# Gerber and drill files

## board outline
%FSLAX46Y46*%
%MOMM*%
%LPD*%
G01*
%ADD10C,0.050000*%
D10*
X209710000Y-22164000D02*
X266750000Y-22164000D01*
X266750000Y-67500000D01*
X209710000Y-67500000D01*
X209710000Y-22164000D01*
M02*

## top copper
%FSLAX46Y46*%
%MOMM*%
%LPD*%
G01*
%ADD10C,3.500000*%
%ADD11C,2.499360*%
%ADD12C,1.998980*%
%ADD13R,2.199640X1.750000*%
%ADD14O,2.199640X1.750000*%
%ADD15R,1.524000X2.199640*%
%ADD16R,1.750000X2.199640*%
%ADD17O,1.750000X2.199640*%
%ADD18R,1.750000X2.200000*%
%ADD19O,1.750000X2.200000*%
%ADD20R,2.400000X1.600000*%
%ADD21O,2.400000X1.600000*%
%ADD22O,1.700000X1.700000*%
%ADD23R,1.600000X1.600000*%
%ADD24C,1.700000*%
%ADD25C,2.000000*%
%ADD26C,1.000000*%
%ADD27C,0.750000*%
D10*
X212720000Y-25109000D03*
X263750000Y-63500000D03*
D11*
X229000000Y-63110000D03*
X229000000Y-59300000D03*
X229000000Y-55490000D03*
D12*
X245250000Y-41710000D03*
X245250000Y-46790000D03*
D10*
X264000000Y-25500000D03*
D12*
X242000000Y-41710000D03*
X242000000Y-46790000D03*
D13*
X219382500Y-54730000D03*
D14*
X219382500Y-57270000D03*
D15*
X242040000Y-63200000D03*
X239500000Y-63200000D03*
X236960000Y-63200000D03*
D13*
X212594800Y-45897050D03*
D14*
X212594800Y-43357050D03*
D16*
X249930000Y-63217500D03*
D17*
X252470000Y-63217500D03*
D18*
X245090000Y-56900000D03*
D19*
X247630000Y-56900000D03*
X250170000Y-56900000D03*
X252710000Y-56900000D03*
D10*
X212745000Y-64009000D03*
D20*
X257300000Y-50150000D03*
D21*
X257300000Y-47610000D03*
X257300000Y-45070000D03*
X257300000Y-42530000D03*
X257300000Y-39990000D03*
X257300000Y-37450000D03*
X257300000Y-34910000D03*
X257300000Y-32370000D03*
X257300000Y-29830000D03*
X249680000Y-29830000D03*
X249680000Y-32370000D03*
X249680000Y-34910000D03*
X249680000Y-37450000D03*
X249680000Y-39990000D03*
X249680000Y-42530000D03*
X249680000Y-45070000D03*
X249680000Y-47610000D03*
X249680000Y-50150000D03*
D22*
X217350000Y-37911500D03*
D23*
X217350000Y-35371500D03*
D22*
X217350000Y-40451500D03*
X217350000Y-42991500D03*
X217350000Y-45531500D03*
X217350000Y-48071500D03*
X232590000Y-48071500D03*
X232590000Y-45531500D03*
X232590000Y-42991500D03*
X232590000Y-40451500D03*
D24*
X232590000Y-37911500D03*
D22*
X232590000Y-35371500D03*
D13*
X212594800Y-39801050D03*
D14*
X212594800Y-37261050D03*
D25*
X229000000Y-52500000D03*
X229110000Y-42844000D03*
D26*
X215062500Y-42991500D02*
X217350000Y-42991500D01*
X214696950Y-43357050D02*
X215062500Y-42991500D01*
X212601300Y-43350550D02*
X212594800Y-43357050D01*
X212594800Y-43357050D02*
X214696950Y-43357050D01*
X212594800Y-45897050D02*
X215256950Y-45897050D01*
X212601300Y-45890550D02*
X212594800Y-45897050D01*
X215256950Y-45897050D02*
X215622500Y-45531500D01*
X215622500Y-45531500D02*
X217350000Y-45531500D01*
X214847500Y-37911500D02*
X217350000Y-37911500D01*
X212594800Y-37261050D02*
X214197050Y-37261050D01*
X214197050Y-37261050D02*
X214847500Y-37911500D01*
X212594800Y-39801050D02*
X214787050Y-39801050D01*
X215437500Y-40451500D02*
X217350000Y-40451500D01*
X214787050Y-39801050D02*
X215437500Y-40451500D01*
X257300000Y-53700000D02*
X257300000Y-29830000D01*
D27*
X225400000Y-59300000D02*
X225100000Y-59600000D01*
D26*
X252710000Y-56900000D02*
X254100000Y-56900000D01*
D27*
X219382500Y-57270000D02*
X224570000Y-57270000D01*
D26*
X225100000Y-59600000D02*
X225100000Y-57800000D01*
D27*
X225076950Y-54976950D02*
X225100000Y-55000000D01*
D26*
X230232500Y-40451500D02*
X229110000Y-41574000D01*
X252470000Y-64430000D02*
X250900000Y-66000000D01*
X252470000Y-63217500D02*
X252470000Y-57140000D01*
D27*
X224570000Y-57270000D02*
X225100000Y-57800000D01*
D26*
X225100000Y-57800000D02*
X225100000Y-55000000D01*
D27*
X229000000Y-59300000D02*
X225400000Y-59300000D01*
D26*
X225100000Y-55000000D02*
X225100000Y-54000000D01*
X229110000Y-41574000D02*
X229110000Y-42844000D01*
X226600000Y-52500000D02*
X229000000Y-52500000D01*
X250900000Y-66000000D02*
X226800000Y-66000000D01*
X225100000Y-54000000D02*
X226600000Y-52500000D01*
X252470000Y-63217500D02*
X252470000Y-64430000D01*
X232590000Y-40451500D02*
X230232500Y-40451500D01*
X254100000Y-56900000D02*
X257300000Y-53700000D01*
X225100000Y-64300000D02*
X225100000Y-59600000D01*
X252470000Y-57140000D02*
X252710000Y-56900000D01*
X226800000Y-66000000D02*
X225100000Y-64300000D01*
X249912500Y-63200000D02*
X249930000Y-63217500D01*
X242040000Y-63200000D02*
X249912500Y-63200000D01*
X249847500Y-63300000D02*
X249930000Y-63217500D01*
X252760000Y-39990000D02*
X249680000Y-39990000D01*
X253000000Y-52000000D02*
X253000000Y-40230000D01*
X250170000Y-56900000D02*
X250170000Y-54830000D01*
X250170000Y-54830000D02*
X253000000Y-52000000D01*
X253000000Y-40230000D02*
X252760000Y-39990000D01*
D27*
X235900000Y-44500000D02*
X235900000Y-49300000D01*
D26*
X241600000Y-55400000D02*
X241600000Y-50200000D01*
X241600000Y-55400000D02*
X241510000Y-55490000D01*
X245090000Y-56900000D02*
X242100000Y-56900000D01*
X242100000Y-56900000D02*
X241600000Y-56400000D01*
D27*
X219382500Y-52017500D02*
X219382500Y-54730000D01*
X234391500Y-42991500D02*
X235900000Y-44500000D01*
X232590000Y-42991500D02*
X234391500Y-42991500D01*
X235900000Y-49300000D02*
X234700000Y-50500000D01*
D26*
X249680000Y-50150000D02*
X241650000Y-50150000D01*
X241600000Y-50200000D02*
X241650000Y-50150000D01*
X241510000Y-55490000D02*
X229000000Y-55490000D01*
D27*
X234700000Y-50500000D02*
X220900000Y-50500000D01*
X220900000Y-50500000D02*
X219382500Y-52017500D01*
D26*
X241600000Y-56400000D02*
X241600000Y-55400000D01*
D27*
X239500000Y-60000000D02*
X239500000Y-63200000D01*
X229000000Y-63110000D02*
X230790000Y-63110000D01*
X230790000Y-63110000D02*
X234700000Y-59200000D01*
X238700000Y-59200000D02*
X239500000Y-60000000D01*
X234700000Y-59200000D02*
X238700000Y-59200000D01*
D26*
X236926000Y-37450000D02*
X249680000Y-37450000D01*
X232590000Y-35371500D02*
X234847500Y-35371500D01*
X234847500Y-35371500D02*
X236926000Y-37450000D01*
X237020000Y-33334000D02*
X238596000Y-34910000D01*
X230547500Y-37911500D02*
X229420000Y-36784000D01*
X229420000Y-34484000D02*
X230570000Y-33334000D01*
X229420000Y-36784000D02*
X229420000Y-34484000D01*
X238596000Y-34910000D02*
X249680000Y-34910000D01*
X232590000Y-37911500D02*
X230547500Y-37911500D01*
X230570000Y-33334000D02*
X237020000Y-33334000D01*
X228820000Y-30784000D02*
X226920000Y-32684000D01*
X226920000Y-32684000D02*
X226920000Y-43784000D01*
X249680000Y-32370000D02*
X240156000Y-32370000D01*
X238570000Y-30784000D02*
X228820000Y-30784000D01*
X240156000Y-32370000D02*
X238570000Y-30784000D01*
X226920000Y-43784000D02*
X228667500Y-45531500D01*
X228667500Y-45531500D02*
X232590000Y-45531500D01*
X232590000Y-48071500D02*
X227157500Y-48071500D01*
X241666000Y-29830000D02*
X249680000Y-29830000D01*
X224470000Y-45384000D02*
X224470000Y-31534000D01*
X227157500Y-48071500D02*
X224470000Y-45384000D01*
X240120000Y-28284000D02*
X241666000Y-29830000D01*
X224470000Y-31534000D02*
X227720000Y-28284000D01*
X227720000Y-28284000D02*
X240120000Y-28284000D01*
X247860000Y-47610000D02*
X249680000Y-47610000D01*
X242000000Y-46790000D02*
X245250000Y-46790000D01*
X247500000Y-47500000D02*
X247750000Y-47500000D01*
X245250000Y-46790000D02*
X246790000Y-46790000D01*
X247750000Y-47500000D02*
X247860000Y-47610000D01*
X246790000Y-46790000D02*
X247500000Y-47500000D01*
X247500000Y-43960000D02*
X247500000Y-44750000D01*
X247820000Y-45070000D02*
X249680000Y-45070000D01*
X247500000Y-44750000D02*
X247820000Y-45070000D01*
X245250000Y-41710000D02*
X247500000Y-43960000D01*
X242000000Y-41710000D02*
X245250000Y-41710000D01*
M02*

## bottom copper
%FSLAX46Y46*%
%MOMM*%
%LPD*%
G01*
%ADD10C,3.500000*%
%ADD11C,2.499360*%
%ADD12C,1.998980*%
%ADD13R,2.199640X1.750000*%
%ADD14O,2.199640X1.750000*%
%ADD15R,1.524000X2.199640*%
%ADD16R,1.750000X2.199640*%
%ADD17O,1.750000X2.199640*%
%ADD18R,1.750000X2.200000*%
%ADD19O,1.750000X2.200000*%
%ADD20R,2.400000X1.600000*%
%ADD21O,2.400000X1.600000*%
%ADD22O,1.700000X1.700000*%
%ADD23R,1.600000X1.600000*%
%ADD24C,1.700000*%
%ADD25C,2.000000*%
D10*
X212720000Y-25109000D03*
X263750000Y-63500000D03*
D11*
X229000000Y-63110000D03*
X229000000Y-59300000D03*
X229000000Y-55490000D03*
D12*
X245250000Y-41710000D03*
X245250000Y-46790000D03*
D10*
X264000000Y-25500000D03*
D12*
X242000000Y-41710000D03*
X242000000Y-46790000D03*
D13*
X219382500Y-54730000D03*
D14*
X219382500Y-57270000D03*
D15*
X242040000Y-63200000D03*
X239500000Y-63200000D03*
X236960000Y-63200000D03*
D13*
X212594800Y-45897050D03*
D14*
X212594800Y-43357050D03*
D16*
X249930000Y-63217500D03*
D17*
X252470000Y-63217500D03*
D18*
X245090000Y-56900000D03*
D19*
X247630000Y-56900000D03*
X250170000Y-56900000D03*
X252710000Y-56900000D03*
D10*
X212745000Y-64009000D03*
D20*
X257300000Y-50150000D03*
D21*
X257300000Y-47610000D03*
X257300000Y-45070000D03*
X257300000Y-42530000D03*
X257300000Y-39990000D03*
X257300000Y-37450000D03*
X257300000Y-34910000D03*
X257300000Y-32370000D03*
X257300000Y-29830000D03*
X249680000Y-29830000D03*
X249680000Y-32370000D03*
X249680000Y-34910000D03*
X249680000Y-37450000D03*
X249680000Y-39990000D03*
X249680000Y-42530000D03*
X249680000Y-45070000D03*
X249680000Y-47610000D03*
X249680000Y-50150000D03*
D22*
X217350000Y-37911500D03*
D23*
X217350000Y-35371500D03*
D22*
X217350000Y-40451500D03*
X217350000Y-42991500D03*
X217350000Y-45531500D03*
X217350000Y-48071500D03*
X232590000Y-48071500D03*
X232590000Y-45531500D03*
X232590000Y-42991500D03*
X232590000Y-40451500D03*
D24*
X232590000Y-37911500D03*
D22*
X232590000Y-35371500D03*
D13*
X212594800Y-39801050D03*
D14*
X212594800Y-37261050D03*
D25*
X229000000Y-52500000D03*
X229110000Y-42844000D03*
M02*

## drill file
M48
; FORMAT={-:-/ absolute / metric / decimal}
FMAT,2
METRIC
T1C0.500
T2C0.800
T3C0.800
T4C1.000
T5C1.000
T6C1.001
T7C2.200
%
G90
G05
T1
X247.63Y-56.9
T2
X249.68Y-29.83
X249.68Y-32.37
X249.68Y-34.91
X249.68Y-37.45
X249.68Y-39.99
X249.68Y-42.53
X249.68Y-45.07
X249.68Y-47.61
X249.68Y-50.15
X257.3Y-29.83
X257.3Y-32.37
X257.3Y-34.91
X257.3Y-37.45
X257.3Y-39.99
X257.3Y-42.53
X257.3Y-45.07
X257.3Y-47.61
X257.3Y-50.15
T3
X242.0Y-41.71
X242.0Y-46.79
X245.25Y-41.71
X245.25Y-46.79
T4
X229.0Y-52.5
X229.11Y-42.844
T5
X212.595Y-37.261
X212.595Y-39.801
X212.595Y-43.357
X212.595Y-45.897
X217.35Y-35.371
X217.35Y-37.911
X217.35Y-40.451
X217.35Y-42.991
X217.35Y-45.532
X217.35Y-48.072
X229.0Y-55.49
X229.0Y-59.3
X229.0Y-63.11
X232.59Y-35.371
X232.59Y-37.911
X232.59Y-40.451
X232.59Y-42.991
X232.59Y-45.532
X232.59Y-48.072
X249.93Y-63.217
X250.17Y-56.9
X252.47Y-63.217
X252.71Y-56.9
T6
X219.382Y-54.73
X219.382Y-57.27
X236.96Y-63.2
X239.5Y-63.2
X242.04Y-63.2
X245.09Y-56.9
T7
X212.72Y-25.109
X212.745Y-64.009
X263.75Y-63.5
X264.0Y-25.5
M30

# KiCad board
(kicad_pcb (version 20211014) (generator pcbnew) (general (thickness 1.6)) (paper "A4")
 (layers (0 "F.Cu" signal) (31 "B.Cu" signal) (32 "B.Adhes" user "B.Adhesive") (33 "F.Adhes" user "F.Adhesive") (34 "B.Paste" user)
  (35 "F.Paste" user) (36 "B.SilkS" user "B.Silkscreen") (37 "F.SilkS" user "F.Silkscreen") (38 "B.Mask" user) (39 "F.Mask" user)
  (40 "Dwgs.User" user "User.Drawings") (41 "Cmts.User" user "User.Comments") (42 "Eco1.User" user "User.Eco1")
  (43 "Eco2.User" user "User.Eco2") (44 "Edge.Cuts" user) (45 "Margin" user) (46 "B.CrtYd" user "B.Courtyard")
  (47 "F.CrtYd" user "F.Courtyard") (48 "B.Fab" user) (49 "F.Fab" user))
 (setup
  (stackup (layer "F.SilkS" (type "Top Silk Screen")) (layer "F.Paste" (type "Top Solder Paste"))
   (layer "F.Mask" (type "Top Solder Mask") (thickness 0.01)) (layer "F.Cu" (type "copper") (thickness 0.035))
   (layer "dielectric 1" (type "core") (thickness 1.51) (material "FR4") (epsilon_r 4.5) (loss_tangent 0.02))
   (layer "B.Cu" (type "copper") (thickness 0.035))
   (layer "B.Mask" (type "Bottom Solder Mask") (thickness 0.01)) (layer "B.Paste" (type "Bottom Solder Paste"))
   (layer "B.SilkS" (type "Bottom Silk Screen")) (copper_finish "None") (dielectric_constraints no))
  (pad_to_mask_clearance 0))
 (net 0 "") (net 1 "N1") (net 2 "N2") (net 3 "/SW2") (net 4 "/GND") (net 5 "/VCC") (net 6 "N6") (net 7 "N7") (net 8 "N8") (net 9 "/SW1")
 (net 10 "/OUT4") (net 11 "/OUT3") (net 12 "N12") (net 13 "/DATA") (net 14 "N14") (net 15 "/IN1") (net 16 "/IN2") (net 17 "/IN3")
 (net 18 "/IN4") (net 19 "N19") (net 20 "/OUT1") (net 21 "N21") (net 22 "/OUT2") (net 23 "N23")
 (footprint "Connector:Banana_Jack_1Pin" (layer "F.Cu") (at 212.72 25.109)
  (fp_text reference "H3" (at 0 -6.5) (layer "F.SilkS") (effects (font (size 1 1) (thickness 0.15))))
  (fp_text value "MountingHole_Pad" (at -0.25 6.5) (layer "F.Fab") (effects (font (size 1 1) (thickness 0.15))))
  (pad "1" thru_hole circle (at 0 0) (size 3.5 3.5) (drill 2.2) (layers *.Cu *.Mask) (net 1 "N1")))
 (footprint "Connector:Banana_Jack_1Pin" (layer "F.Cu") (at 263.75 63.5)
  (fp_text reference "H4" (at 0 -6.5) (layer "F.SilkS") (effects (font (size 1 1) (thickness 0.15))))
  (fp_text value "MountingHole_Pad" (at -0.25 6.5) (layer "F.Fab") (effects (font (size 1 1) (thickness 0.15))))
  (pad "1" thru_hole circle (at 0 0) (size 3.5 3.5) (drill 2.2) (layers *.Cu *.Mask) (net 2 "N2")))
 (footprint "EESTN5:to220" (layer "F.Cu") (at 229 59.3 90)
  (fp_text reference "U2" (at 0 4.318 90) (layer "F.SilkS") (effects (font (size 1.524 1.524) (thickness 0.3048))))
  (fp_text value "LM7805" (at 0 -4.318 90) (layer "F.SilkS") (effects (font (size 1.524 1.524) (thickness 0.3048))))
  (pad "1" thru_hole circle locked (at -3.81 0 90) (size 2.49936 2.49936) (drill 1) (layers *.Cu *.Mask "F.SilkS") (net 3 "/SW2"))
  (pad "2" thru_hole circle locked (at 0 0 90) (size 2.49936 2.49936) (drill 1) (layers *.Cu *.Mask "F.SilkS") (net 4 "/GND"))
  (pad "3" thru_hole circle locked (at 3.81 0 90) (size 2.49936 2.49936) (drill 1) (layers *.Cu *.Mask "F.SilkS") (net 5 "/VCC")))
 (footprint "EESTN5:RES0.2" (layer "F.Cu") (at 245.25 44.25 -90)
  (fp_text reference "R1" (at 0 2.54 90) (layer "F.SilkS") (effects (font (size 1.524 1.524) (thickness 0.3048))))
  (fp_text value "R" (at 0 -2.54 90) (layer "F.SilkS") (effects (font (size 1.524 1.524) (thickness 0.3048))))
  (pad "1" thru_hole circle locked (at -2.54 0 270) (size 1.99898 1.99898) (drill 0.8001) (layers *.Cu *.Mask "F.SilkS") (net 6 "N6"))
  (pad "2" thru_hole circle locked (at 2.54 0 270) (size 1.99898 1.99898) (drill 0.8001) (layers *.Cu *.Mask "F.SilkS") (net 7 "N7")))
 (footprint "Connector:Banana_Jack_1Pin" (layer "F.Cu") (at 264 25.5)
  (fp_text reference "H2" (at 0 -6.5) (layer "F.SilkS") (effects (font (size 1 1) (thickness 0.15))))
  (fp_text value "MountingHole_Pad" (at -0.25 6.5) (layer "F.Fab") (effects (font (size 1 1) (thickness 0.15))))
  (pad "1" thru_hole circle (at 0 0) (size 3.5 3.5) (drill 2.2) (layers *.Cu *.Mask) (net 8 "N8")))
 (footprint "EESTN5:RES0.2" (layer "F.Cu") (at 242 44.25 -90)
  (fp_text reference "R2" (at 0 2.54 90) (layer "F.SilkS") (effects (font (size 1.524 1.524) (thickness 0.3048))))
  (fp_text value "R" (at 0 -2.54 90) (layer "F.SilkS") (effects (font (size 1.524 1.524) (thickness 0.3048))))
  (pad "1" thru_hole circle locked (at -2.54 0 270) (size 1.99898 1.99898) (drill 0.8001) (layers *.Cu *.Mask "F.SilkS") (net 6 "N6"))
  (pad "2" thru_hole circle locked (at 2.54 0 270) (size 1.99898 1.99898) (drill 0.8001) (layers *.Cu *.Mask "F.SilkS") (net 7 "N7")))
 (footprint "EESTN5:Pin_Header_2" (layer "F.Cu") (at 219.7 56 -90)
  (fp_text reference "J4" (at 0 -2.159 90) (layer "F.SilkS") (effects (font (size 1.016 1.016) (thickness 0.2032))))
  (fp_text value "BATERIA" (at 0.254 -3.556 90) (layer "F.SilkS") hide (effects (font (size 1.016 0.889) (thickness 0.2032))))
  (pad "1" thru_hole rect locked (at -1.27 0.3175 270) (size 1.75 2.19964) (drill 1.00076) (layers *.Cu *.Mask "F.SilkS") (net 5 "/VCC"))
  (pad "2" thru_hole oval locked (at 1.27 0.3175 270) (size 1.75 2.19964) (drill 1.00076) (layers *.Cu *.Mask "F.SilkS") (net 4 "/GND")))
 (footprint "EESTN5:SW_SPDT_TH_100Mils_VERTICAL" (layer "F.Cu") (at 239.5 63.2 180)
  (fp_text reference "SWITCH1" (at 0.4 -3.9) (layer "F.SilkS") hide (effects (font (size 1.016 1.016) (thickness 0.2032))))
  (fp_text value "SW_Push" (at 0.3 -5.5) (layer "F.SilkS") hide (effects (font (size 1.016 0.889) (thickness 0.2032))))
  (pad "1" thru_hole rect locked (at -2.54 0 180) (size 1.524 2.19964) (drill 1.00076) (layers *.Cu *.Mask "F.SilkS") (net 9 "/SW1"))
  (pad "2" thru_hole rect locked (at 0 0 180) (size 1.524 2.19964) (drill 1.00076) (layers *.Cu *.Mask "F.SilkS") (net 3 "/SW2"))
  (pad "3" thru_hole rect locked (at 2.54 0 180) (size 1.524 2.19964) (drill 1.00076) (layers *.Cu *.Mask "F.SilkS")))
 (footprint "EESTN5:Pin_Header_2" (layer "F.Cu") (at 212.2773 44.62705 90)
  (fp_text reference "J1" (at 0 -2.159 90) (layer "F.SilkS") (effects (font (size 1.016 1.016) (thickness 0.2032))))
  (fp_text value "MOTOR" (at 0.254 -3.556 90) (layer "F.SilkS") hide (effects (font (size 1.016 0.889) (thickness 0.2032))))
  (pad "1" thru_hole rect locked (at -1.27 0.3175 90) (size 1.75 2.19964) (drill 1) (layers *.Cu *.Mask "F.SilkS") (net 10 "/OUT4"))
  (pad "2" thru_hole oval locked (at 1.27 0.3175 90) (size 1.75 2.19964) (drill 1) (layers *.Cu *.Mask "F.SilkS") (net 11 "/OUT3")))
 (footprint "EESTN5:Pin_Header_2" (layer "F.Cu") (at 251.2 62.9)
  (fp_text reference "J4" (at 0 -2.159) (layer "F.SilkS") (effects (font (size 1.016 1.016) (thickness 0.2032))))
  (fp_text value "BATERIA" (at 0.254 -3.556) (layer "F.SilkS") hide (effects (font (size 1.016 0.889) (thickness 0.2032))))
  (pad "1" thru_hole rect locked (at -1.27 0.3175) (size 1.75 2.19964) (drill 1) (layers *.Cu *.Mask "F.SilkS") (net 9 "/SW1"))
  (pad "2" thru_hole oval locked (at 1.27 0.3175) (size 1.75 2.19964) (drill 1) (layers *.Cu *.Mask "F.SilkS") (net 4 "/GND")))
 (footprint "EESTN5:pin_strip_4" (layer "F.Cu") (at 248.9 56.9)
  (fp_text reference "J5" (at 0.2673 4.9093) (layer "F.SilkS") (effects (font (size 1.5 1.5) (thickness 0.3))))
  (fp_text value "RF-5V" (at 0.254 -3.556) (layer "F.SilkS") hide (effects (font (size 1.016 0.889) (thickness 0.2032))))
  (pad "1" thru_hole rect locked (at -3.81 0) (size 1.75 2.2) (drill 1.00076) (layers *.Cu *.Mask "F.SilkS") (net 5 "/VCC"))
  (pad "2" thru_hole oval locked (at -1.27 0) (size 1.75 2.2) (drill 0.5) (layers *.Cu *.Mask "F.SilkS") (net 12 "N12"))
  (pad "3" thru_hole oval locked (at 1.27 0) (size 1.75 2.2) (drill 1) (layers *.Cu *.Mask "F.SilkS") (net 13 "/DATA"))
  (pad "4" thru_hole oval locked (at 3.81 0) (size 1.75 2.2) (drill 1) (layers *.Cu *.Mask "F.SilkS") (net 4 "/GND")))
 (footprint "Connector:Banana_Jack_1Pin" (layer "F.Cu") (at 212.745 64.009)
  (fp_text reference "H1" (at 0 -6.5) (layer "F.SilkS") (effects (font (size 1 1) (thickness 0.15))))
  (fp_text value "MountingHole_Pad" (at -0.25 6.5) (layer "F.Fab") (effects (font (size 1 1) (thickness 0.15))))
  (pad "1" thru_hole circle (at 0 0) (size 3.5 3.5) (drill 2.2) (layers *.Cu *.Mask) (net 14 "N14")))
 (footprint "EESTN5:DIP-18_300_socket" (layer "F.Cu") (at 257.3 50.15 180)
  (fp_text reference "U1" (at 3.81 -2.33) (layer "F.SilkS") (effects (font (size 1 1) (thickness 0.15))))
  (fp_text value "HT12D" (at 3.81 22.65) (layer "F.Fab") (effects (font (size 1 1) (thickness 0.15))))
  (pad "1" thru_hole rect locked (at 0 0 180) (size 2.4 1.6) (drill 0.8) (layers *.Cu *.Mask) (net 4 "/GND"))
  (pad "2" thru_hole oval locked (at 0 2.54 180) (size 2.4 1.6) (drill 0.8) (layers *.Cu *.Mask) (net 4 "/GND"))
  (pad "3" thru_hole oval locked (at 0 5.08 180) (size 2.4 1.6) (drill 0.8) (layers *.Cu *.Mask) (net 4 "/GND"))
  (pad "4" thru_hole oval locked (at 0 7.62 180) (size 2.4 1.6) (drill 0.8) (layers *.Cu *.Mask) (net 4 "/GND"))
  (pad "5" thru_hole oval locked (at 0 10.16 180) (size 2.4 1.6) (drill 0.8) (layers *.Cu *.Mask) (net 4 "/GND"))
  (pad "6" thru_hole oval locked (at 0 12.7 180) (size 2.4 1.6) (drill 0.8) (layers *.Cu *.Mask) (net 4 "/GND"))
  (pad "7" thru_hole oval locked (at 0 15.24 180) (size 2.4 1.6) (drill 0.8) (layers *.Cu *.Mask) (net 4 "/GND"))
  (pad "8" thru_hole oval locked (at 0 17.78 180) (size 2.4 1.6) (drill 0.8) (layers *.Cu *.Mask) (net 4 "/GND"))
  (pad "9" thru_hole oval locked (at 0 20.32 180) (size 2.4 1.6) (drill 0.8) (layers *.Cu *.Mask) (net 4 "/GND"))
  (pad "10" thru_hole oval locked (at 7.62 20.32 180) (size 2.4 1.6) (drill 0.8) (layers *.Cu *.Mask) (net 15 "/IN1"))
  (pad "11" thru_hole oval locked (at 7.62 17.78 180) (size 2.4 1.6) (drill 0.8) (layers *.Cu *.Mask) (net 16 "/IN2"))
  (pad "12" thru_hole oval locked (at 7.62 15.24 180) (size 2.4 1.6) (drill 0.8) (layers *.Cu *.Mask) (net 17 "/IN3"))
  (pad "13" thru_hole oval locked (at 7.62 12.7 180) (size 2.4 1.6) (drill 0.8) (layers *.Cu *.Mask) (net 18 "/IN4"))
  (pad "14" thru_hole oval locked (at 7.62 10.16 180) (size 2.4 1.6) (drill 0.8) (layers *.Cu *.Mask) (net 13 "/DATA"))
  (pad "15" thru_hole oval locked (at 7.62 7.62 180) (size 2.4 1.6) (drill 0.8) (layers *.Cu *.Mask) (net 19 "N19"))
  (pad "16" thru_hole oval locked (at 7.62 5.08 180) (size 2.4 1.6) (drill 0.8) (layers *.Cu *.Mask) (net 6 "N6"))
  (pad "17" thru_hole oval locked (at 7.62 2.54 180) (size 2.4 1.6) (drill 0.8) (layers *.Cu *.Mask) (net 7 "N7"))
  (pad "18" thru_hole oval locked (at 7.62 0 180) (size 2.4 1.6) (drill 0.8) (layers *.Cu *.Mask) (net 5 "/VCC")))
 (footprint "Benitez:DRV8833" (layer "F.Cu") (at 217.35 35.3715)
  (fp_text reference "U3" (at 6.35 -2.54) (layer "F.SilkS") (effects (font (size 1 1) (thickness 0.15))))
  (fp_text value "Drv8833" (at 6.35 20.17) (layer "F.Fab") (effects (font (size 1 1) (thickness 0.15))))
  (pad "1" thru_hole oval (at 0 2.54) (size 1.7 1.7) (drill 1) (layers *.Cu *.Mask) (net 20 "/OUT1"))
  (pad "1" thru_hole rect (at 0 0) (size 1.6 1.6) (drill 1) (layers *.Cu *.Mask) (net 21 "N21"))
  (pad "3" thru_hole oval (at 0 5.08) (size 1.7 1.7) (drill 1) (layers *.Cu *.Mask "B.SilkS") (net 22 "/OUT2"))
  (pad "4" thru_hole oval (at 0 7.62) (size 1.7 1.7) (drill 1) (layers *.Cu *.Mask) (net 11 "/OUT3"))
  (pad "5" thru_hole oval (at 0 10.16) (size 1.7 1.7) (drill 1) (layers *.Cu *.Mask) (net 10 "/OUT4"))
  (pad "6" thru_hole oval (at 0 12.7) (size 1.7 1.7) (drill 1) (layers *.Cu *.Mask) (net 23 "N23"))
  (pad "7" thru_hole oval (at 15.24 12.7) (size 1.7 1.7) (drill 1) (layers *.Cu *.Mask) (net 15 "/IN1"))
  (pad "8" thru_hole oval (at 15.24 10.16) (size 1.7 1.7) (drill 1) (layers *.Cu *.Mask) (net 16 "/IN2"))
  (pad "9" thru_hole oval (at 15.24 7.62) (size 1.7 1.7) (drill 1) (layers *.Cu *.Mask) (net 5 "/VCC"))
  (pad "10" thru_hole oval (at 15.24 5.08) (size 1.7 1.7) (drill 1) (layers *.Cu *.Mask) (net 4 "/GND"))
  (pad "11" thru_hole circle (at 15.24 2.54) (size 1.7 1.7) (drill 1) (layers *.Cu *.Mask) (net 17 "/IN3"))
  (pad "12" thru_hole oval (at 15.24 0) (size 1.7 1.7) (drill 1) (layers *.Cu *.Mask) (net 18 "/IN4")))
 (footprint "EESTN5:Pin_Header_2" (layer "F.Cu") (at 212.2773 38.53105 90)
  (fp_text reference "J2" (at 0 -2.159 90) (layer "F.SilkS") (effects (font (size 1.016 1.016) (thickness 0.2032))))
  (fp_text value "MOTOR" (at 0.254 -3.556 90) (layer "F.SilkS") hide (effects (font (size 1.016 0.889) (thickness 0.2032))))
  (pad "1" thru_hole rect locked (at -1.27 0.3175 90) (size 1.75 2.19964) (drill 1) (layers *.Cu *.Mask "F.SilkS") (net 22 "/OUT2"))
  (pad "2" thru_hole oval locked (at 1.27 0.3175 90) (size 1.75 2.19964) (drill 1) (layers *.Cu *.Mask "F.SilkS") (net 20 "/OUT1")))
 (gr_rect (start 266.75 67.5) (end 209.71 22.164) (layer "Edge.Cuts") (width 0.05) (fill none))
 (segment (start 215.0625 42.9915) (end 217.35 42.9915) (width 1) (layer "F.Cu") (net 11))
 (segment (start 214.69695 43.35705) (end 215.0625 42.9915) (width 1) (layer "F.Cu") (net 11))
 (segment (start 212.6013 43.35055) (end 212.5948 43.35705) (width 1) (layer "F.Cu") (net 11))
 (segment (start 212.5948 43.35705) (end 214.69695 43.35705) (width 1) (layer "F.Cu") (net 11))
 (segment (start 212.5948 45.89705) (end 215.25695 45.89705) (width 1) (layer "F.Cu") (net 10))
 (segment (start 212.6013 45.89055) (end 212.5948 45.89705) (width 1) (layer "F.Cu") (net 10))
 (segment (start 215.25695 45.89705) (end 215.6225 45.5315) (width 1) (layer "F.Cu") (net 10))
 (segment (start 215.6225 45.5315) (end 217.35 45.5315) (width 1) (layer "F.Cu") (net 10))
 (segment (start 214.8475 37.9115) (end 217.35 37.9115) (width 1) (layer "F.Cu") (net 20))
 (segment (start 212.5948 37.26105) (end 214.19705 37.26105) (width 1) (layer "F.Cu") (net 20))
 (segment (start 214.19705 37.26105) (end 214.8475 37.9115) (width 1) (layer "F.Cu") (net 20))
 (segment (start 212.5948 39.80105) (end 214.78705 39.80105) (width 1) (layer "F.Cu") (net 22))
 (segment (start 215.4375 40.4515) (end 217.35 40.4515) (width 1) (layer "F.Cu") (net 22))
 (segment (start 214.78705 39.80105) (end 215.4375 40.4515) (width 1) (layer "F.Cu") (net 22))
 (segment (start 257.3 53.7) (end 257.3 29.83) (width 1) (layer "F.Cu") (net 4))
 (segment (start 225.4 59.3) (end 225.1 59.6) (width 0.75) (layer "F.Cu") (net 4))
 (segment (start 252.71 56.9) (end 254.1 56.9) (width 1) (layer "F.Cu") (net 4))
 (segment (start 219.3825 57.27) (end 224.57 57.27) (width 0.75) (layer "F.Cu") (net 4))
 (segment (start 225.1 59.6) (end 225.1 57.8) (width 1) (layer "F.Cu") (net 4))
 (segment (start 225.07695 54.97695) (end 225.1 55) (width 0.75) (layer "F.Cu") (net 4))
 (segment (start 230.2325 40.4515) (end 229.11 41.574) (width 1) (layer "F.Cu") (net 4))
 (segment (start 252.47 64.43) (end 250.9 66) (width 1) (layer "F.Cu") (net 4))
 (segment (start 252.47 63.2175) (end 252.47 57.14) (width 1) (layer "F.Cu") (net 4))
 (segment (start 224.57 57.27) (end 225.1 57.8) (width 0.75) (layer "F.Cu") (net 4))
 (segment (start 225.1 57.8) (end 225.1 55) (width 1) (layer "F.Cu") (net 4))
 (segment (start 229 59.3) (end 225.4 59.3) (width 0.75) (layer "F.Cu") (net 4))
 (segment (start 225.1 55) (end 225.1 54) (width 1) (layer "F.Cu") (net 4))
 (segment (start 229.11 41.574) (end 229.11 42.844) (width 1) (layer "F.Cu") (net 4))
 (segment (start 226.6 52.5) (end 229 52.5) (width 1) (layer "F.Cu") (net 4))
 (segment (start 250.9 66) (end 226.8 66) (width 1) (layer "F.Cu") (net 4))
 (segment (start 225.1 54) (end 226.6 52.5) (width 1) (layer "F.Cu") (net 4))
 (segment (start 252.47 63.2175) (end 252.47 64.43) (width 1) (layer "F.Cu") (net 4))
 (segment (start 232.59 40.4515) (end 230.2325 40.4515) (width 1) (layer "F.Cu") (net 4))
 (segment (start 254.1 56.9) (end 257.3 53.7) (width 1) (layer "F.Cu") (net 4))
 (segment (start 225.1 64.3) (end 225.1 59.6) (width 1) (layer "F.Cu") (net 4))
 (segment (start 252.47 57.14) (end 252.71 56.9) (width 1) (layer "F.Cu") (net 4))
 (segment (start 226.8 66) (end 225.1 64.3) (width 1) (layer "F.Cu") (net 4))
 (via (at 229 52.5) (size 2) (drill 1) (layers "F.Cu" "B.Cu") (free) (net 4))
 (via (at 229.11 42.844) (size 2) (drill 1) (layers "F.Cu" "B.Cu") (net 4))
 (segment (start 249.9125 63.2) (end 249.93 63.2175) (width 1) (layer "F.Cu") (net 9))
 (segment (start 242.04 63.2) (end 249.9125 63.2) (width 1) (layer "F.Cu") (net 9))
 (segment (start 249.8475 63.3) (end 249.93 63.2175) (width 1) (layer "F.Cu") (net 9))
 (segment (start 252.76 39.99) (end 249.68 39.99) (width 1) (layer "F.Cu") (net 13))
 (segment (start 253 52) (end 253 40.23) (width 1) (layer "F.Cu") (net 13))
 (segment (start 250.17 56.9) (end 250.17 54.83) (width 1) (layer "F.Cu") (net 13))
 (segment (start 250.17 54.83) (end 253 52) (width 1) (layer "F.Cu") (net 13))
 (segment (start 253 40.23) (end 252.76 39.99) (width 1) (layer "F.Cu") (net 13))
 (segment (start 235.9 44.5) (end 235.9 49.3) (width 0.75) (layer "F.Cu") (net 5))
 (segment (start 241.6 55.4) (end 241.6 50.2) (width 1) (layer "F.Cu") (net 5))
 (segment (start 241.6 55.4) (end 241.51 55.49) (width 1) (layer "F.Cu") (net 5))
 (segment (start 245.09 56.9) (end 242.1 56.9) (width 1) (layer "F.Cu") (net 5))
 (segment (start 242.1 56.9) (end 241.6 56.4) (width 1) (layer "F.Cu") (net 5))
 (segment (start 219.3825 52.0175) (end 219.3825 54.73) (width 0.75) (layer "F.Cu") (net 5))
 (segment (start 234.3915 42.9915) (end 235.9 44.5) (width 0.75) (layer "F.Cu") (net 5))
 (segment (start 232.59 42.9915) (end 234.3915 42.9915) (width 0.75) (layer "F.Cu") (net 5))
 (segment (start 235.9 49.3) (end 234.7 50.5) (width 0.75) (layer "F.Cu") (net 5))
 (segment (start 249.68 50.15) (end 241.65 50.15) (width 1) (layer "F.Cu") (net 5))
 (segment (start 241.6 50.2) (end 241.65 50.15) (width 1) (layer "F.Cu") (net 5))
 (segment (start 241.51 55.49) (end 229 55.49) (width 1) (layer "F.Cu") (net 5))
 (segment (start 234.7 50.5) (end 220.9 50.5) (width 0.75) (layer "F.Cu") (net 5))
 (segment (start 220.9 50.5) (end 219.3825 52.0175) (width 0.75) (layer "F.Cu") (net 5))
 (segment (start 241.6 56.4) (end 241.6 55.4) (width 1) (layer "F.Cu") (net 5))
 (segment (start 239.5 60) (end 239.5 63.2) (width 0.75) (layer "F.Cu") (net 3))
 (segment (start 229 63.11) (end 230.79 63.11) (width 0.75) (layer "F.Cu") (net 3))
 (segment (start 230.79 63.11) (end 234.7 59.2) (width 0.75) (layer "F.Cu") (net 3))
 (segment (start 238.7 59.2) (end 239.5 60) (width 0.75) (layer "F.Cu") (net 3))
 (segment (start 234.7 59.2) (end 238.7 59.2) (width 0.75) (layer "F.Cu") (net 3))
 (segment (start 236.926 37.45) (end 249.68 37.45) (width 1) (layer "F.Cu") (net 18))
 (segment (start 232.59 35.3715) (end 234.8475 35.3715) (width 1) (layer "F.Cu") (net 18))
 (segment (start 234.8475 35.3715) (end 236.926 37.45) (width 1) (layer "F.Cu") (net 18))
 (segment (start 237.02 33.334) (end 238.596 34.91) (width 1) (layer "F.Cu") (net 17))
 (segment (start 230.5475 37.9115) (end 229.42 36.784) (width 1) (layer "F.Cu") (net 17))
 (segment (start 229.42 34.484) (end 230.57 33.334) (width 1) (layer "F.Cu") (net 17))
 (segment (start 229.42 36.784) (end 229.42 34.484) (width 1) (layer "F.Cu") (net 17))
 (segment (start 238.596 34.91) (end 249.68 34.91) (width 1) (layer "F.Cu") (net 17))
 (segment (start 232.59 37.9115) (end 230.5475 37.9115) (width 1) (layer "F.Cu") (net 17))
 (segment (start 230.57 33.334) (end 237.02 33.334) (width 1) (layer "F.Cu") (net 17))
 (segment (start 228.82 30.784) (end 226.92 32.684) (width 1) (layer "F.Cu") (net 16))
 (segment (start 226.92 32.684) (end 226.92 43.784) (width 1) (layer "F.Cu") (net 16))
 (segment (start 249.68 32.37) (end 240.156 32.37) (width 1) (layer "F.Cu") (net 16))
 (segment (start 238.57 30.784) (end 228.82 30.784) (width 1) (layer "F.Cu") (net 16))
 (segment (start 240.156 32.37) (end 238.57 30.784) (width 1) (layer "F.Cu") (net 16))
 (segment (start 226.92 43.784) (end 228.6675 45.5315) (width 1) (layer "F.Cu") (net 16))
 (segment (start 228.6675 45.5315) (end 232.59 45.5315) (width 1) (layer "F.Cu") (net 16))
 (segment (start 232.59 48.0715) (end 227.1575 48.0715) (width 1) (layer "F.Cu") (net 15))
 (segment (start 241.666 29.83) (end 249.68 29.83) (width 1) (layer "F.Cu") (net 15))
 (segment (start 224.47 45.384) (end 224.47 31.534) (width 1) (layer "F.Cu") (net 15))
 (segment (start 227.1575 48.0715) (end 224.47 45.384) (width 1) (layer "F.Cu") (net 15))
 (segment (start 240.12 28.284) (end 241.666 29.83) (width 1) (layer "F.Cu") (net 15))
 (segment (start 224.47 31.534) (end 227.72 28.284) (width 1) (layer "F.Cu") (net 15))
 (segment (start 227.72 28.284) (end 240.12 28.284) (width 1) (layer "F.Cu") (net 15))
 (segment (start 247.86 47.61) (end 249.68 47.61) (width 1) (layer "F.Cu") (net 7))
 (segment (start 242 46.79) (end 245.25 46.79) (width 1) (layer "F.Cu") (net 7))
 (segment (start 247.5 47.5) (end 247.75 47.5) (width 1) (layer "F.Cu") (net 7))
 (segment (start 245.25 46.79) (end 246.79 46.79) (width 1) (layer "F.Cu") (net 7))
 (segment (start 247.75 47.5) (end 247.86 47.61) (width 1) (layer "F.Cu") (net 7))
 (segment (start 246.79 46.79) (end 247.5 47.5) (width 1) (layer "F.Cu") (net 7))
 (segment (start 247.5 43.96) (end 247.5 44.75) (width 1) (layer "F.Cu") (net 6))
 (segment (start 247.82 45.07) (end 249.68 45.07) (width 1) (layer "F.Cu") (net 6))
 (segment (start 247.5 44.75) (end 247.82 45.07) (width 1) (layer "F.Cu") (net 6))
 (segment (start 245.25 41.71) (end 247.5 43.96) (width 1) (layer "F.Cu") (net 6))
 (segment (start 242 41.71) (end 245.25 41.71) (width 1) (layer "F.Cu") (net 6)))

